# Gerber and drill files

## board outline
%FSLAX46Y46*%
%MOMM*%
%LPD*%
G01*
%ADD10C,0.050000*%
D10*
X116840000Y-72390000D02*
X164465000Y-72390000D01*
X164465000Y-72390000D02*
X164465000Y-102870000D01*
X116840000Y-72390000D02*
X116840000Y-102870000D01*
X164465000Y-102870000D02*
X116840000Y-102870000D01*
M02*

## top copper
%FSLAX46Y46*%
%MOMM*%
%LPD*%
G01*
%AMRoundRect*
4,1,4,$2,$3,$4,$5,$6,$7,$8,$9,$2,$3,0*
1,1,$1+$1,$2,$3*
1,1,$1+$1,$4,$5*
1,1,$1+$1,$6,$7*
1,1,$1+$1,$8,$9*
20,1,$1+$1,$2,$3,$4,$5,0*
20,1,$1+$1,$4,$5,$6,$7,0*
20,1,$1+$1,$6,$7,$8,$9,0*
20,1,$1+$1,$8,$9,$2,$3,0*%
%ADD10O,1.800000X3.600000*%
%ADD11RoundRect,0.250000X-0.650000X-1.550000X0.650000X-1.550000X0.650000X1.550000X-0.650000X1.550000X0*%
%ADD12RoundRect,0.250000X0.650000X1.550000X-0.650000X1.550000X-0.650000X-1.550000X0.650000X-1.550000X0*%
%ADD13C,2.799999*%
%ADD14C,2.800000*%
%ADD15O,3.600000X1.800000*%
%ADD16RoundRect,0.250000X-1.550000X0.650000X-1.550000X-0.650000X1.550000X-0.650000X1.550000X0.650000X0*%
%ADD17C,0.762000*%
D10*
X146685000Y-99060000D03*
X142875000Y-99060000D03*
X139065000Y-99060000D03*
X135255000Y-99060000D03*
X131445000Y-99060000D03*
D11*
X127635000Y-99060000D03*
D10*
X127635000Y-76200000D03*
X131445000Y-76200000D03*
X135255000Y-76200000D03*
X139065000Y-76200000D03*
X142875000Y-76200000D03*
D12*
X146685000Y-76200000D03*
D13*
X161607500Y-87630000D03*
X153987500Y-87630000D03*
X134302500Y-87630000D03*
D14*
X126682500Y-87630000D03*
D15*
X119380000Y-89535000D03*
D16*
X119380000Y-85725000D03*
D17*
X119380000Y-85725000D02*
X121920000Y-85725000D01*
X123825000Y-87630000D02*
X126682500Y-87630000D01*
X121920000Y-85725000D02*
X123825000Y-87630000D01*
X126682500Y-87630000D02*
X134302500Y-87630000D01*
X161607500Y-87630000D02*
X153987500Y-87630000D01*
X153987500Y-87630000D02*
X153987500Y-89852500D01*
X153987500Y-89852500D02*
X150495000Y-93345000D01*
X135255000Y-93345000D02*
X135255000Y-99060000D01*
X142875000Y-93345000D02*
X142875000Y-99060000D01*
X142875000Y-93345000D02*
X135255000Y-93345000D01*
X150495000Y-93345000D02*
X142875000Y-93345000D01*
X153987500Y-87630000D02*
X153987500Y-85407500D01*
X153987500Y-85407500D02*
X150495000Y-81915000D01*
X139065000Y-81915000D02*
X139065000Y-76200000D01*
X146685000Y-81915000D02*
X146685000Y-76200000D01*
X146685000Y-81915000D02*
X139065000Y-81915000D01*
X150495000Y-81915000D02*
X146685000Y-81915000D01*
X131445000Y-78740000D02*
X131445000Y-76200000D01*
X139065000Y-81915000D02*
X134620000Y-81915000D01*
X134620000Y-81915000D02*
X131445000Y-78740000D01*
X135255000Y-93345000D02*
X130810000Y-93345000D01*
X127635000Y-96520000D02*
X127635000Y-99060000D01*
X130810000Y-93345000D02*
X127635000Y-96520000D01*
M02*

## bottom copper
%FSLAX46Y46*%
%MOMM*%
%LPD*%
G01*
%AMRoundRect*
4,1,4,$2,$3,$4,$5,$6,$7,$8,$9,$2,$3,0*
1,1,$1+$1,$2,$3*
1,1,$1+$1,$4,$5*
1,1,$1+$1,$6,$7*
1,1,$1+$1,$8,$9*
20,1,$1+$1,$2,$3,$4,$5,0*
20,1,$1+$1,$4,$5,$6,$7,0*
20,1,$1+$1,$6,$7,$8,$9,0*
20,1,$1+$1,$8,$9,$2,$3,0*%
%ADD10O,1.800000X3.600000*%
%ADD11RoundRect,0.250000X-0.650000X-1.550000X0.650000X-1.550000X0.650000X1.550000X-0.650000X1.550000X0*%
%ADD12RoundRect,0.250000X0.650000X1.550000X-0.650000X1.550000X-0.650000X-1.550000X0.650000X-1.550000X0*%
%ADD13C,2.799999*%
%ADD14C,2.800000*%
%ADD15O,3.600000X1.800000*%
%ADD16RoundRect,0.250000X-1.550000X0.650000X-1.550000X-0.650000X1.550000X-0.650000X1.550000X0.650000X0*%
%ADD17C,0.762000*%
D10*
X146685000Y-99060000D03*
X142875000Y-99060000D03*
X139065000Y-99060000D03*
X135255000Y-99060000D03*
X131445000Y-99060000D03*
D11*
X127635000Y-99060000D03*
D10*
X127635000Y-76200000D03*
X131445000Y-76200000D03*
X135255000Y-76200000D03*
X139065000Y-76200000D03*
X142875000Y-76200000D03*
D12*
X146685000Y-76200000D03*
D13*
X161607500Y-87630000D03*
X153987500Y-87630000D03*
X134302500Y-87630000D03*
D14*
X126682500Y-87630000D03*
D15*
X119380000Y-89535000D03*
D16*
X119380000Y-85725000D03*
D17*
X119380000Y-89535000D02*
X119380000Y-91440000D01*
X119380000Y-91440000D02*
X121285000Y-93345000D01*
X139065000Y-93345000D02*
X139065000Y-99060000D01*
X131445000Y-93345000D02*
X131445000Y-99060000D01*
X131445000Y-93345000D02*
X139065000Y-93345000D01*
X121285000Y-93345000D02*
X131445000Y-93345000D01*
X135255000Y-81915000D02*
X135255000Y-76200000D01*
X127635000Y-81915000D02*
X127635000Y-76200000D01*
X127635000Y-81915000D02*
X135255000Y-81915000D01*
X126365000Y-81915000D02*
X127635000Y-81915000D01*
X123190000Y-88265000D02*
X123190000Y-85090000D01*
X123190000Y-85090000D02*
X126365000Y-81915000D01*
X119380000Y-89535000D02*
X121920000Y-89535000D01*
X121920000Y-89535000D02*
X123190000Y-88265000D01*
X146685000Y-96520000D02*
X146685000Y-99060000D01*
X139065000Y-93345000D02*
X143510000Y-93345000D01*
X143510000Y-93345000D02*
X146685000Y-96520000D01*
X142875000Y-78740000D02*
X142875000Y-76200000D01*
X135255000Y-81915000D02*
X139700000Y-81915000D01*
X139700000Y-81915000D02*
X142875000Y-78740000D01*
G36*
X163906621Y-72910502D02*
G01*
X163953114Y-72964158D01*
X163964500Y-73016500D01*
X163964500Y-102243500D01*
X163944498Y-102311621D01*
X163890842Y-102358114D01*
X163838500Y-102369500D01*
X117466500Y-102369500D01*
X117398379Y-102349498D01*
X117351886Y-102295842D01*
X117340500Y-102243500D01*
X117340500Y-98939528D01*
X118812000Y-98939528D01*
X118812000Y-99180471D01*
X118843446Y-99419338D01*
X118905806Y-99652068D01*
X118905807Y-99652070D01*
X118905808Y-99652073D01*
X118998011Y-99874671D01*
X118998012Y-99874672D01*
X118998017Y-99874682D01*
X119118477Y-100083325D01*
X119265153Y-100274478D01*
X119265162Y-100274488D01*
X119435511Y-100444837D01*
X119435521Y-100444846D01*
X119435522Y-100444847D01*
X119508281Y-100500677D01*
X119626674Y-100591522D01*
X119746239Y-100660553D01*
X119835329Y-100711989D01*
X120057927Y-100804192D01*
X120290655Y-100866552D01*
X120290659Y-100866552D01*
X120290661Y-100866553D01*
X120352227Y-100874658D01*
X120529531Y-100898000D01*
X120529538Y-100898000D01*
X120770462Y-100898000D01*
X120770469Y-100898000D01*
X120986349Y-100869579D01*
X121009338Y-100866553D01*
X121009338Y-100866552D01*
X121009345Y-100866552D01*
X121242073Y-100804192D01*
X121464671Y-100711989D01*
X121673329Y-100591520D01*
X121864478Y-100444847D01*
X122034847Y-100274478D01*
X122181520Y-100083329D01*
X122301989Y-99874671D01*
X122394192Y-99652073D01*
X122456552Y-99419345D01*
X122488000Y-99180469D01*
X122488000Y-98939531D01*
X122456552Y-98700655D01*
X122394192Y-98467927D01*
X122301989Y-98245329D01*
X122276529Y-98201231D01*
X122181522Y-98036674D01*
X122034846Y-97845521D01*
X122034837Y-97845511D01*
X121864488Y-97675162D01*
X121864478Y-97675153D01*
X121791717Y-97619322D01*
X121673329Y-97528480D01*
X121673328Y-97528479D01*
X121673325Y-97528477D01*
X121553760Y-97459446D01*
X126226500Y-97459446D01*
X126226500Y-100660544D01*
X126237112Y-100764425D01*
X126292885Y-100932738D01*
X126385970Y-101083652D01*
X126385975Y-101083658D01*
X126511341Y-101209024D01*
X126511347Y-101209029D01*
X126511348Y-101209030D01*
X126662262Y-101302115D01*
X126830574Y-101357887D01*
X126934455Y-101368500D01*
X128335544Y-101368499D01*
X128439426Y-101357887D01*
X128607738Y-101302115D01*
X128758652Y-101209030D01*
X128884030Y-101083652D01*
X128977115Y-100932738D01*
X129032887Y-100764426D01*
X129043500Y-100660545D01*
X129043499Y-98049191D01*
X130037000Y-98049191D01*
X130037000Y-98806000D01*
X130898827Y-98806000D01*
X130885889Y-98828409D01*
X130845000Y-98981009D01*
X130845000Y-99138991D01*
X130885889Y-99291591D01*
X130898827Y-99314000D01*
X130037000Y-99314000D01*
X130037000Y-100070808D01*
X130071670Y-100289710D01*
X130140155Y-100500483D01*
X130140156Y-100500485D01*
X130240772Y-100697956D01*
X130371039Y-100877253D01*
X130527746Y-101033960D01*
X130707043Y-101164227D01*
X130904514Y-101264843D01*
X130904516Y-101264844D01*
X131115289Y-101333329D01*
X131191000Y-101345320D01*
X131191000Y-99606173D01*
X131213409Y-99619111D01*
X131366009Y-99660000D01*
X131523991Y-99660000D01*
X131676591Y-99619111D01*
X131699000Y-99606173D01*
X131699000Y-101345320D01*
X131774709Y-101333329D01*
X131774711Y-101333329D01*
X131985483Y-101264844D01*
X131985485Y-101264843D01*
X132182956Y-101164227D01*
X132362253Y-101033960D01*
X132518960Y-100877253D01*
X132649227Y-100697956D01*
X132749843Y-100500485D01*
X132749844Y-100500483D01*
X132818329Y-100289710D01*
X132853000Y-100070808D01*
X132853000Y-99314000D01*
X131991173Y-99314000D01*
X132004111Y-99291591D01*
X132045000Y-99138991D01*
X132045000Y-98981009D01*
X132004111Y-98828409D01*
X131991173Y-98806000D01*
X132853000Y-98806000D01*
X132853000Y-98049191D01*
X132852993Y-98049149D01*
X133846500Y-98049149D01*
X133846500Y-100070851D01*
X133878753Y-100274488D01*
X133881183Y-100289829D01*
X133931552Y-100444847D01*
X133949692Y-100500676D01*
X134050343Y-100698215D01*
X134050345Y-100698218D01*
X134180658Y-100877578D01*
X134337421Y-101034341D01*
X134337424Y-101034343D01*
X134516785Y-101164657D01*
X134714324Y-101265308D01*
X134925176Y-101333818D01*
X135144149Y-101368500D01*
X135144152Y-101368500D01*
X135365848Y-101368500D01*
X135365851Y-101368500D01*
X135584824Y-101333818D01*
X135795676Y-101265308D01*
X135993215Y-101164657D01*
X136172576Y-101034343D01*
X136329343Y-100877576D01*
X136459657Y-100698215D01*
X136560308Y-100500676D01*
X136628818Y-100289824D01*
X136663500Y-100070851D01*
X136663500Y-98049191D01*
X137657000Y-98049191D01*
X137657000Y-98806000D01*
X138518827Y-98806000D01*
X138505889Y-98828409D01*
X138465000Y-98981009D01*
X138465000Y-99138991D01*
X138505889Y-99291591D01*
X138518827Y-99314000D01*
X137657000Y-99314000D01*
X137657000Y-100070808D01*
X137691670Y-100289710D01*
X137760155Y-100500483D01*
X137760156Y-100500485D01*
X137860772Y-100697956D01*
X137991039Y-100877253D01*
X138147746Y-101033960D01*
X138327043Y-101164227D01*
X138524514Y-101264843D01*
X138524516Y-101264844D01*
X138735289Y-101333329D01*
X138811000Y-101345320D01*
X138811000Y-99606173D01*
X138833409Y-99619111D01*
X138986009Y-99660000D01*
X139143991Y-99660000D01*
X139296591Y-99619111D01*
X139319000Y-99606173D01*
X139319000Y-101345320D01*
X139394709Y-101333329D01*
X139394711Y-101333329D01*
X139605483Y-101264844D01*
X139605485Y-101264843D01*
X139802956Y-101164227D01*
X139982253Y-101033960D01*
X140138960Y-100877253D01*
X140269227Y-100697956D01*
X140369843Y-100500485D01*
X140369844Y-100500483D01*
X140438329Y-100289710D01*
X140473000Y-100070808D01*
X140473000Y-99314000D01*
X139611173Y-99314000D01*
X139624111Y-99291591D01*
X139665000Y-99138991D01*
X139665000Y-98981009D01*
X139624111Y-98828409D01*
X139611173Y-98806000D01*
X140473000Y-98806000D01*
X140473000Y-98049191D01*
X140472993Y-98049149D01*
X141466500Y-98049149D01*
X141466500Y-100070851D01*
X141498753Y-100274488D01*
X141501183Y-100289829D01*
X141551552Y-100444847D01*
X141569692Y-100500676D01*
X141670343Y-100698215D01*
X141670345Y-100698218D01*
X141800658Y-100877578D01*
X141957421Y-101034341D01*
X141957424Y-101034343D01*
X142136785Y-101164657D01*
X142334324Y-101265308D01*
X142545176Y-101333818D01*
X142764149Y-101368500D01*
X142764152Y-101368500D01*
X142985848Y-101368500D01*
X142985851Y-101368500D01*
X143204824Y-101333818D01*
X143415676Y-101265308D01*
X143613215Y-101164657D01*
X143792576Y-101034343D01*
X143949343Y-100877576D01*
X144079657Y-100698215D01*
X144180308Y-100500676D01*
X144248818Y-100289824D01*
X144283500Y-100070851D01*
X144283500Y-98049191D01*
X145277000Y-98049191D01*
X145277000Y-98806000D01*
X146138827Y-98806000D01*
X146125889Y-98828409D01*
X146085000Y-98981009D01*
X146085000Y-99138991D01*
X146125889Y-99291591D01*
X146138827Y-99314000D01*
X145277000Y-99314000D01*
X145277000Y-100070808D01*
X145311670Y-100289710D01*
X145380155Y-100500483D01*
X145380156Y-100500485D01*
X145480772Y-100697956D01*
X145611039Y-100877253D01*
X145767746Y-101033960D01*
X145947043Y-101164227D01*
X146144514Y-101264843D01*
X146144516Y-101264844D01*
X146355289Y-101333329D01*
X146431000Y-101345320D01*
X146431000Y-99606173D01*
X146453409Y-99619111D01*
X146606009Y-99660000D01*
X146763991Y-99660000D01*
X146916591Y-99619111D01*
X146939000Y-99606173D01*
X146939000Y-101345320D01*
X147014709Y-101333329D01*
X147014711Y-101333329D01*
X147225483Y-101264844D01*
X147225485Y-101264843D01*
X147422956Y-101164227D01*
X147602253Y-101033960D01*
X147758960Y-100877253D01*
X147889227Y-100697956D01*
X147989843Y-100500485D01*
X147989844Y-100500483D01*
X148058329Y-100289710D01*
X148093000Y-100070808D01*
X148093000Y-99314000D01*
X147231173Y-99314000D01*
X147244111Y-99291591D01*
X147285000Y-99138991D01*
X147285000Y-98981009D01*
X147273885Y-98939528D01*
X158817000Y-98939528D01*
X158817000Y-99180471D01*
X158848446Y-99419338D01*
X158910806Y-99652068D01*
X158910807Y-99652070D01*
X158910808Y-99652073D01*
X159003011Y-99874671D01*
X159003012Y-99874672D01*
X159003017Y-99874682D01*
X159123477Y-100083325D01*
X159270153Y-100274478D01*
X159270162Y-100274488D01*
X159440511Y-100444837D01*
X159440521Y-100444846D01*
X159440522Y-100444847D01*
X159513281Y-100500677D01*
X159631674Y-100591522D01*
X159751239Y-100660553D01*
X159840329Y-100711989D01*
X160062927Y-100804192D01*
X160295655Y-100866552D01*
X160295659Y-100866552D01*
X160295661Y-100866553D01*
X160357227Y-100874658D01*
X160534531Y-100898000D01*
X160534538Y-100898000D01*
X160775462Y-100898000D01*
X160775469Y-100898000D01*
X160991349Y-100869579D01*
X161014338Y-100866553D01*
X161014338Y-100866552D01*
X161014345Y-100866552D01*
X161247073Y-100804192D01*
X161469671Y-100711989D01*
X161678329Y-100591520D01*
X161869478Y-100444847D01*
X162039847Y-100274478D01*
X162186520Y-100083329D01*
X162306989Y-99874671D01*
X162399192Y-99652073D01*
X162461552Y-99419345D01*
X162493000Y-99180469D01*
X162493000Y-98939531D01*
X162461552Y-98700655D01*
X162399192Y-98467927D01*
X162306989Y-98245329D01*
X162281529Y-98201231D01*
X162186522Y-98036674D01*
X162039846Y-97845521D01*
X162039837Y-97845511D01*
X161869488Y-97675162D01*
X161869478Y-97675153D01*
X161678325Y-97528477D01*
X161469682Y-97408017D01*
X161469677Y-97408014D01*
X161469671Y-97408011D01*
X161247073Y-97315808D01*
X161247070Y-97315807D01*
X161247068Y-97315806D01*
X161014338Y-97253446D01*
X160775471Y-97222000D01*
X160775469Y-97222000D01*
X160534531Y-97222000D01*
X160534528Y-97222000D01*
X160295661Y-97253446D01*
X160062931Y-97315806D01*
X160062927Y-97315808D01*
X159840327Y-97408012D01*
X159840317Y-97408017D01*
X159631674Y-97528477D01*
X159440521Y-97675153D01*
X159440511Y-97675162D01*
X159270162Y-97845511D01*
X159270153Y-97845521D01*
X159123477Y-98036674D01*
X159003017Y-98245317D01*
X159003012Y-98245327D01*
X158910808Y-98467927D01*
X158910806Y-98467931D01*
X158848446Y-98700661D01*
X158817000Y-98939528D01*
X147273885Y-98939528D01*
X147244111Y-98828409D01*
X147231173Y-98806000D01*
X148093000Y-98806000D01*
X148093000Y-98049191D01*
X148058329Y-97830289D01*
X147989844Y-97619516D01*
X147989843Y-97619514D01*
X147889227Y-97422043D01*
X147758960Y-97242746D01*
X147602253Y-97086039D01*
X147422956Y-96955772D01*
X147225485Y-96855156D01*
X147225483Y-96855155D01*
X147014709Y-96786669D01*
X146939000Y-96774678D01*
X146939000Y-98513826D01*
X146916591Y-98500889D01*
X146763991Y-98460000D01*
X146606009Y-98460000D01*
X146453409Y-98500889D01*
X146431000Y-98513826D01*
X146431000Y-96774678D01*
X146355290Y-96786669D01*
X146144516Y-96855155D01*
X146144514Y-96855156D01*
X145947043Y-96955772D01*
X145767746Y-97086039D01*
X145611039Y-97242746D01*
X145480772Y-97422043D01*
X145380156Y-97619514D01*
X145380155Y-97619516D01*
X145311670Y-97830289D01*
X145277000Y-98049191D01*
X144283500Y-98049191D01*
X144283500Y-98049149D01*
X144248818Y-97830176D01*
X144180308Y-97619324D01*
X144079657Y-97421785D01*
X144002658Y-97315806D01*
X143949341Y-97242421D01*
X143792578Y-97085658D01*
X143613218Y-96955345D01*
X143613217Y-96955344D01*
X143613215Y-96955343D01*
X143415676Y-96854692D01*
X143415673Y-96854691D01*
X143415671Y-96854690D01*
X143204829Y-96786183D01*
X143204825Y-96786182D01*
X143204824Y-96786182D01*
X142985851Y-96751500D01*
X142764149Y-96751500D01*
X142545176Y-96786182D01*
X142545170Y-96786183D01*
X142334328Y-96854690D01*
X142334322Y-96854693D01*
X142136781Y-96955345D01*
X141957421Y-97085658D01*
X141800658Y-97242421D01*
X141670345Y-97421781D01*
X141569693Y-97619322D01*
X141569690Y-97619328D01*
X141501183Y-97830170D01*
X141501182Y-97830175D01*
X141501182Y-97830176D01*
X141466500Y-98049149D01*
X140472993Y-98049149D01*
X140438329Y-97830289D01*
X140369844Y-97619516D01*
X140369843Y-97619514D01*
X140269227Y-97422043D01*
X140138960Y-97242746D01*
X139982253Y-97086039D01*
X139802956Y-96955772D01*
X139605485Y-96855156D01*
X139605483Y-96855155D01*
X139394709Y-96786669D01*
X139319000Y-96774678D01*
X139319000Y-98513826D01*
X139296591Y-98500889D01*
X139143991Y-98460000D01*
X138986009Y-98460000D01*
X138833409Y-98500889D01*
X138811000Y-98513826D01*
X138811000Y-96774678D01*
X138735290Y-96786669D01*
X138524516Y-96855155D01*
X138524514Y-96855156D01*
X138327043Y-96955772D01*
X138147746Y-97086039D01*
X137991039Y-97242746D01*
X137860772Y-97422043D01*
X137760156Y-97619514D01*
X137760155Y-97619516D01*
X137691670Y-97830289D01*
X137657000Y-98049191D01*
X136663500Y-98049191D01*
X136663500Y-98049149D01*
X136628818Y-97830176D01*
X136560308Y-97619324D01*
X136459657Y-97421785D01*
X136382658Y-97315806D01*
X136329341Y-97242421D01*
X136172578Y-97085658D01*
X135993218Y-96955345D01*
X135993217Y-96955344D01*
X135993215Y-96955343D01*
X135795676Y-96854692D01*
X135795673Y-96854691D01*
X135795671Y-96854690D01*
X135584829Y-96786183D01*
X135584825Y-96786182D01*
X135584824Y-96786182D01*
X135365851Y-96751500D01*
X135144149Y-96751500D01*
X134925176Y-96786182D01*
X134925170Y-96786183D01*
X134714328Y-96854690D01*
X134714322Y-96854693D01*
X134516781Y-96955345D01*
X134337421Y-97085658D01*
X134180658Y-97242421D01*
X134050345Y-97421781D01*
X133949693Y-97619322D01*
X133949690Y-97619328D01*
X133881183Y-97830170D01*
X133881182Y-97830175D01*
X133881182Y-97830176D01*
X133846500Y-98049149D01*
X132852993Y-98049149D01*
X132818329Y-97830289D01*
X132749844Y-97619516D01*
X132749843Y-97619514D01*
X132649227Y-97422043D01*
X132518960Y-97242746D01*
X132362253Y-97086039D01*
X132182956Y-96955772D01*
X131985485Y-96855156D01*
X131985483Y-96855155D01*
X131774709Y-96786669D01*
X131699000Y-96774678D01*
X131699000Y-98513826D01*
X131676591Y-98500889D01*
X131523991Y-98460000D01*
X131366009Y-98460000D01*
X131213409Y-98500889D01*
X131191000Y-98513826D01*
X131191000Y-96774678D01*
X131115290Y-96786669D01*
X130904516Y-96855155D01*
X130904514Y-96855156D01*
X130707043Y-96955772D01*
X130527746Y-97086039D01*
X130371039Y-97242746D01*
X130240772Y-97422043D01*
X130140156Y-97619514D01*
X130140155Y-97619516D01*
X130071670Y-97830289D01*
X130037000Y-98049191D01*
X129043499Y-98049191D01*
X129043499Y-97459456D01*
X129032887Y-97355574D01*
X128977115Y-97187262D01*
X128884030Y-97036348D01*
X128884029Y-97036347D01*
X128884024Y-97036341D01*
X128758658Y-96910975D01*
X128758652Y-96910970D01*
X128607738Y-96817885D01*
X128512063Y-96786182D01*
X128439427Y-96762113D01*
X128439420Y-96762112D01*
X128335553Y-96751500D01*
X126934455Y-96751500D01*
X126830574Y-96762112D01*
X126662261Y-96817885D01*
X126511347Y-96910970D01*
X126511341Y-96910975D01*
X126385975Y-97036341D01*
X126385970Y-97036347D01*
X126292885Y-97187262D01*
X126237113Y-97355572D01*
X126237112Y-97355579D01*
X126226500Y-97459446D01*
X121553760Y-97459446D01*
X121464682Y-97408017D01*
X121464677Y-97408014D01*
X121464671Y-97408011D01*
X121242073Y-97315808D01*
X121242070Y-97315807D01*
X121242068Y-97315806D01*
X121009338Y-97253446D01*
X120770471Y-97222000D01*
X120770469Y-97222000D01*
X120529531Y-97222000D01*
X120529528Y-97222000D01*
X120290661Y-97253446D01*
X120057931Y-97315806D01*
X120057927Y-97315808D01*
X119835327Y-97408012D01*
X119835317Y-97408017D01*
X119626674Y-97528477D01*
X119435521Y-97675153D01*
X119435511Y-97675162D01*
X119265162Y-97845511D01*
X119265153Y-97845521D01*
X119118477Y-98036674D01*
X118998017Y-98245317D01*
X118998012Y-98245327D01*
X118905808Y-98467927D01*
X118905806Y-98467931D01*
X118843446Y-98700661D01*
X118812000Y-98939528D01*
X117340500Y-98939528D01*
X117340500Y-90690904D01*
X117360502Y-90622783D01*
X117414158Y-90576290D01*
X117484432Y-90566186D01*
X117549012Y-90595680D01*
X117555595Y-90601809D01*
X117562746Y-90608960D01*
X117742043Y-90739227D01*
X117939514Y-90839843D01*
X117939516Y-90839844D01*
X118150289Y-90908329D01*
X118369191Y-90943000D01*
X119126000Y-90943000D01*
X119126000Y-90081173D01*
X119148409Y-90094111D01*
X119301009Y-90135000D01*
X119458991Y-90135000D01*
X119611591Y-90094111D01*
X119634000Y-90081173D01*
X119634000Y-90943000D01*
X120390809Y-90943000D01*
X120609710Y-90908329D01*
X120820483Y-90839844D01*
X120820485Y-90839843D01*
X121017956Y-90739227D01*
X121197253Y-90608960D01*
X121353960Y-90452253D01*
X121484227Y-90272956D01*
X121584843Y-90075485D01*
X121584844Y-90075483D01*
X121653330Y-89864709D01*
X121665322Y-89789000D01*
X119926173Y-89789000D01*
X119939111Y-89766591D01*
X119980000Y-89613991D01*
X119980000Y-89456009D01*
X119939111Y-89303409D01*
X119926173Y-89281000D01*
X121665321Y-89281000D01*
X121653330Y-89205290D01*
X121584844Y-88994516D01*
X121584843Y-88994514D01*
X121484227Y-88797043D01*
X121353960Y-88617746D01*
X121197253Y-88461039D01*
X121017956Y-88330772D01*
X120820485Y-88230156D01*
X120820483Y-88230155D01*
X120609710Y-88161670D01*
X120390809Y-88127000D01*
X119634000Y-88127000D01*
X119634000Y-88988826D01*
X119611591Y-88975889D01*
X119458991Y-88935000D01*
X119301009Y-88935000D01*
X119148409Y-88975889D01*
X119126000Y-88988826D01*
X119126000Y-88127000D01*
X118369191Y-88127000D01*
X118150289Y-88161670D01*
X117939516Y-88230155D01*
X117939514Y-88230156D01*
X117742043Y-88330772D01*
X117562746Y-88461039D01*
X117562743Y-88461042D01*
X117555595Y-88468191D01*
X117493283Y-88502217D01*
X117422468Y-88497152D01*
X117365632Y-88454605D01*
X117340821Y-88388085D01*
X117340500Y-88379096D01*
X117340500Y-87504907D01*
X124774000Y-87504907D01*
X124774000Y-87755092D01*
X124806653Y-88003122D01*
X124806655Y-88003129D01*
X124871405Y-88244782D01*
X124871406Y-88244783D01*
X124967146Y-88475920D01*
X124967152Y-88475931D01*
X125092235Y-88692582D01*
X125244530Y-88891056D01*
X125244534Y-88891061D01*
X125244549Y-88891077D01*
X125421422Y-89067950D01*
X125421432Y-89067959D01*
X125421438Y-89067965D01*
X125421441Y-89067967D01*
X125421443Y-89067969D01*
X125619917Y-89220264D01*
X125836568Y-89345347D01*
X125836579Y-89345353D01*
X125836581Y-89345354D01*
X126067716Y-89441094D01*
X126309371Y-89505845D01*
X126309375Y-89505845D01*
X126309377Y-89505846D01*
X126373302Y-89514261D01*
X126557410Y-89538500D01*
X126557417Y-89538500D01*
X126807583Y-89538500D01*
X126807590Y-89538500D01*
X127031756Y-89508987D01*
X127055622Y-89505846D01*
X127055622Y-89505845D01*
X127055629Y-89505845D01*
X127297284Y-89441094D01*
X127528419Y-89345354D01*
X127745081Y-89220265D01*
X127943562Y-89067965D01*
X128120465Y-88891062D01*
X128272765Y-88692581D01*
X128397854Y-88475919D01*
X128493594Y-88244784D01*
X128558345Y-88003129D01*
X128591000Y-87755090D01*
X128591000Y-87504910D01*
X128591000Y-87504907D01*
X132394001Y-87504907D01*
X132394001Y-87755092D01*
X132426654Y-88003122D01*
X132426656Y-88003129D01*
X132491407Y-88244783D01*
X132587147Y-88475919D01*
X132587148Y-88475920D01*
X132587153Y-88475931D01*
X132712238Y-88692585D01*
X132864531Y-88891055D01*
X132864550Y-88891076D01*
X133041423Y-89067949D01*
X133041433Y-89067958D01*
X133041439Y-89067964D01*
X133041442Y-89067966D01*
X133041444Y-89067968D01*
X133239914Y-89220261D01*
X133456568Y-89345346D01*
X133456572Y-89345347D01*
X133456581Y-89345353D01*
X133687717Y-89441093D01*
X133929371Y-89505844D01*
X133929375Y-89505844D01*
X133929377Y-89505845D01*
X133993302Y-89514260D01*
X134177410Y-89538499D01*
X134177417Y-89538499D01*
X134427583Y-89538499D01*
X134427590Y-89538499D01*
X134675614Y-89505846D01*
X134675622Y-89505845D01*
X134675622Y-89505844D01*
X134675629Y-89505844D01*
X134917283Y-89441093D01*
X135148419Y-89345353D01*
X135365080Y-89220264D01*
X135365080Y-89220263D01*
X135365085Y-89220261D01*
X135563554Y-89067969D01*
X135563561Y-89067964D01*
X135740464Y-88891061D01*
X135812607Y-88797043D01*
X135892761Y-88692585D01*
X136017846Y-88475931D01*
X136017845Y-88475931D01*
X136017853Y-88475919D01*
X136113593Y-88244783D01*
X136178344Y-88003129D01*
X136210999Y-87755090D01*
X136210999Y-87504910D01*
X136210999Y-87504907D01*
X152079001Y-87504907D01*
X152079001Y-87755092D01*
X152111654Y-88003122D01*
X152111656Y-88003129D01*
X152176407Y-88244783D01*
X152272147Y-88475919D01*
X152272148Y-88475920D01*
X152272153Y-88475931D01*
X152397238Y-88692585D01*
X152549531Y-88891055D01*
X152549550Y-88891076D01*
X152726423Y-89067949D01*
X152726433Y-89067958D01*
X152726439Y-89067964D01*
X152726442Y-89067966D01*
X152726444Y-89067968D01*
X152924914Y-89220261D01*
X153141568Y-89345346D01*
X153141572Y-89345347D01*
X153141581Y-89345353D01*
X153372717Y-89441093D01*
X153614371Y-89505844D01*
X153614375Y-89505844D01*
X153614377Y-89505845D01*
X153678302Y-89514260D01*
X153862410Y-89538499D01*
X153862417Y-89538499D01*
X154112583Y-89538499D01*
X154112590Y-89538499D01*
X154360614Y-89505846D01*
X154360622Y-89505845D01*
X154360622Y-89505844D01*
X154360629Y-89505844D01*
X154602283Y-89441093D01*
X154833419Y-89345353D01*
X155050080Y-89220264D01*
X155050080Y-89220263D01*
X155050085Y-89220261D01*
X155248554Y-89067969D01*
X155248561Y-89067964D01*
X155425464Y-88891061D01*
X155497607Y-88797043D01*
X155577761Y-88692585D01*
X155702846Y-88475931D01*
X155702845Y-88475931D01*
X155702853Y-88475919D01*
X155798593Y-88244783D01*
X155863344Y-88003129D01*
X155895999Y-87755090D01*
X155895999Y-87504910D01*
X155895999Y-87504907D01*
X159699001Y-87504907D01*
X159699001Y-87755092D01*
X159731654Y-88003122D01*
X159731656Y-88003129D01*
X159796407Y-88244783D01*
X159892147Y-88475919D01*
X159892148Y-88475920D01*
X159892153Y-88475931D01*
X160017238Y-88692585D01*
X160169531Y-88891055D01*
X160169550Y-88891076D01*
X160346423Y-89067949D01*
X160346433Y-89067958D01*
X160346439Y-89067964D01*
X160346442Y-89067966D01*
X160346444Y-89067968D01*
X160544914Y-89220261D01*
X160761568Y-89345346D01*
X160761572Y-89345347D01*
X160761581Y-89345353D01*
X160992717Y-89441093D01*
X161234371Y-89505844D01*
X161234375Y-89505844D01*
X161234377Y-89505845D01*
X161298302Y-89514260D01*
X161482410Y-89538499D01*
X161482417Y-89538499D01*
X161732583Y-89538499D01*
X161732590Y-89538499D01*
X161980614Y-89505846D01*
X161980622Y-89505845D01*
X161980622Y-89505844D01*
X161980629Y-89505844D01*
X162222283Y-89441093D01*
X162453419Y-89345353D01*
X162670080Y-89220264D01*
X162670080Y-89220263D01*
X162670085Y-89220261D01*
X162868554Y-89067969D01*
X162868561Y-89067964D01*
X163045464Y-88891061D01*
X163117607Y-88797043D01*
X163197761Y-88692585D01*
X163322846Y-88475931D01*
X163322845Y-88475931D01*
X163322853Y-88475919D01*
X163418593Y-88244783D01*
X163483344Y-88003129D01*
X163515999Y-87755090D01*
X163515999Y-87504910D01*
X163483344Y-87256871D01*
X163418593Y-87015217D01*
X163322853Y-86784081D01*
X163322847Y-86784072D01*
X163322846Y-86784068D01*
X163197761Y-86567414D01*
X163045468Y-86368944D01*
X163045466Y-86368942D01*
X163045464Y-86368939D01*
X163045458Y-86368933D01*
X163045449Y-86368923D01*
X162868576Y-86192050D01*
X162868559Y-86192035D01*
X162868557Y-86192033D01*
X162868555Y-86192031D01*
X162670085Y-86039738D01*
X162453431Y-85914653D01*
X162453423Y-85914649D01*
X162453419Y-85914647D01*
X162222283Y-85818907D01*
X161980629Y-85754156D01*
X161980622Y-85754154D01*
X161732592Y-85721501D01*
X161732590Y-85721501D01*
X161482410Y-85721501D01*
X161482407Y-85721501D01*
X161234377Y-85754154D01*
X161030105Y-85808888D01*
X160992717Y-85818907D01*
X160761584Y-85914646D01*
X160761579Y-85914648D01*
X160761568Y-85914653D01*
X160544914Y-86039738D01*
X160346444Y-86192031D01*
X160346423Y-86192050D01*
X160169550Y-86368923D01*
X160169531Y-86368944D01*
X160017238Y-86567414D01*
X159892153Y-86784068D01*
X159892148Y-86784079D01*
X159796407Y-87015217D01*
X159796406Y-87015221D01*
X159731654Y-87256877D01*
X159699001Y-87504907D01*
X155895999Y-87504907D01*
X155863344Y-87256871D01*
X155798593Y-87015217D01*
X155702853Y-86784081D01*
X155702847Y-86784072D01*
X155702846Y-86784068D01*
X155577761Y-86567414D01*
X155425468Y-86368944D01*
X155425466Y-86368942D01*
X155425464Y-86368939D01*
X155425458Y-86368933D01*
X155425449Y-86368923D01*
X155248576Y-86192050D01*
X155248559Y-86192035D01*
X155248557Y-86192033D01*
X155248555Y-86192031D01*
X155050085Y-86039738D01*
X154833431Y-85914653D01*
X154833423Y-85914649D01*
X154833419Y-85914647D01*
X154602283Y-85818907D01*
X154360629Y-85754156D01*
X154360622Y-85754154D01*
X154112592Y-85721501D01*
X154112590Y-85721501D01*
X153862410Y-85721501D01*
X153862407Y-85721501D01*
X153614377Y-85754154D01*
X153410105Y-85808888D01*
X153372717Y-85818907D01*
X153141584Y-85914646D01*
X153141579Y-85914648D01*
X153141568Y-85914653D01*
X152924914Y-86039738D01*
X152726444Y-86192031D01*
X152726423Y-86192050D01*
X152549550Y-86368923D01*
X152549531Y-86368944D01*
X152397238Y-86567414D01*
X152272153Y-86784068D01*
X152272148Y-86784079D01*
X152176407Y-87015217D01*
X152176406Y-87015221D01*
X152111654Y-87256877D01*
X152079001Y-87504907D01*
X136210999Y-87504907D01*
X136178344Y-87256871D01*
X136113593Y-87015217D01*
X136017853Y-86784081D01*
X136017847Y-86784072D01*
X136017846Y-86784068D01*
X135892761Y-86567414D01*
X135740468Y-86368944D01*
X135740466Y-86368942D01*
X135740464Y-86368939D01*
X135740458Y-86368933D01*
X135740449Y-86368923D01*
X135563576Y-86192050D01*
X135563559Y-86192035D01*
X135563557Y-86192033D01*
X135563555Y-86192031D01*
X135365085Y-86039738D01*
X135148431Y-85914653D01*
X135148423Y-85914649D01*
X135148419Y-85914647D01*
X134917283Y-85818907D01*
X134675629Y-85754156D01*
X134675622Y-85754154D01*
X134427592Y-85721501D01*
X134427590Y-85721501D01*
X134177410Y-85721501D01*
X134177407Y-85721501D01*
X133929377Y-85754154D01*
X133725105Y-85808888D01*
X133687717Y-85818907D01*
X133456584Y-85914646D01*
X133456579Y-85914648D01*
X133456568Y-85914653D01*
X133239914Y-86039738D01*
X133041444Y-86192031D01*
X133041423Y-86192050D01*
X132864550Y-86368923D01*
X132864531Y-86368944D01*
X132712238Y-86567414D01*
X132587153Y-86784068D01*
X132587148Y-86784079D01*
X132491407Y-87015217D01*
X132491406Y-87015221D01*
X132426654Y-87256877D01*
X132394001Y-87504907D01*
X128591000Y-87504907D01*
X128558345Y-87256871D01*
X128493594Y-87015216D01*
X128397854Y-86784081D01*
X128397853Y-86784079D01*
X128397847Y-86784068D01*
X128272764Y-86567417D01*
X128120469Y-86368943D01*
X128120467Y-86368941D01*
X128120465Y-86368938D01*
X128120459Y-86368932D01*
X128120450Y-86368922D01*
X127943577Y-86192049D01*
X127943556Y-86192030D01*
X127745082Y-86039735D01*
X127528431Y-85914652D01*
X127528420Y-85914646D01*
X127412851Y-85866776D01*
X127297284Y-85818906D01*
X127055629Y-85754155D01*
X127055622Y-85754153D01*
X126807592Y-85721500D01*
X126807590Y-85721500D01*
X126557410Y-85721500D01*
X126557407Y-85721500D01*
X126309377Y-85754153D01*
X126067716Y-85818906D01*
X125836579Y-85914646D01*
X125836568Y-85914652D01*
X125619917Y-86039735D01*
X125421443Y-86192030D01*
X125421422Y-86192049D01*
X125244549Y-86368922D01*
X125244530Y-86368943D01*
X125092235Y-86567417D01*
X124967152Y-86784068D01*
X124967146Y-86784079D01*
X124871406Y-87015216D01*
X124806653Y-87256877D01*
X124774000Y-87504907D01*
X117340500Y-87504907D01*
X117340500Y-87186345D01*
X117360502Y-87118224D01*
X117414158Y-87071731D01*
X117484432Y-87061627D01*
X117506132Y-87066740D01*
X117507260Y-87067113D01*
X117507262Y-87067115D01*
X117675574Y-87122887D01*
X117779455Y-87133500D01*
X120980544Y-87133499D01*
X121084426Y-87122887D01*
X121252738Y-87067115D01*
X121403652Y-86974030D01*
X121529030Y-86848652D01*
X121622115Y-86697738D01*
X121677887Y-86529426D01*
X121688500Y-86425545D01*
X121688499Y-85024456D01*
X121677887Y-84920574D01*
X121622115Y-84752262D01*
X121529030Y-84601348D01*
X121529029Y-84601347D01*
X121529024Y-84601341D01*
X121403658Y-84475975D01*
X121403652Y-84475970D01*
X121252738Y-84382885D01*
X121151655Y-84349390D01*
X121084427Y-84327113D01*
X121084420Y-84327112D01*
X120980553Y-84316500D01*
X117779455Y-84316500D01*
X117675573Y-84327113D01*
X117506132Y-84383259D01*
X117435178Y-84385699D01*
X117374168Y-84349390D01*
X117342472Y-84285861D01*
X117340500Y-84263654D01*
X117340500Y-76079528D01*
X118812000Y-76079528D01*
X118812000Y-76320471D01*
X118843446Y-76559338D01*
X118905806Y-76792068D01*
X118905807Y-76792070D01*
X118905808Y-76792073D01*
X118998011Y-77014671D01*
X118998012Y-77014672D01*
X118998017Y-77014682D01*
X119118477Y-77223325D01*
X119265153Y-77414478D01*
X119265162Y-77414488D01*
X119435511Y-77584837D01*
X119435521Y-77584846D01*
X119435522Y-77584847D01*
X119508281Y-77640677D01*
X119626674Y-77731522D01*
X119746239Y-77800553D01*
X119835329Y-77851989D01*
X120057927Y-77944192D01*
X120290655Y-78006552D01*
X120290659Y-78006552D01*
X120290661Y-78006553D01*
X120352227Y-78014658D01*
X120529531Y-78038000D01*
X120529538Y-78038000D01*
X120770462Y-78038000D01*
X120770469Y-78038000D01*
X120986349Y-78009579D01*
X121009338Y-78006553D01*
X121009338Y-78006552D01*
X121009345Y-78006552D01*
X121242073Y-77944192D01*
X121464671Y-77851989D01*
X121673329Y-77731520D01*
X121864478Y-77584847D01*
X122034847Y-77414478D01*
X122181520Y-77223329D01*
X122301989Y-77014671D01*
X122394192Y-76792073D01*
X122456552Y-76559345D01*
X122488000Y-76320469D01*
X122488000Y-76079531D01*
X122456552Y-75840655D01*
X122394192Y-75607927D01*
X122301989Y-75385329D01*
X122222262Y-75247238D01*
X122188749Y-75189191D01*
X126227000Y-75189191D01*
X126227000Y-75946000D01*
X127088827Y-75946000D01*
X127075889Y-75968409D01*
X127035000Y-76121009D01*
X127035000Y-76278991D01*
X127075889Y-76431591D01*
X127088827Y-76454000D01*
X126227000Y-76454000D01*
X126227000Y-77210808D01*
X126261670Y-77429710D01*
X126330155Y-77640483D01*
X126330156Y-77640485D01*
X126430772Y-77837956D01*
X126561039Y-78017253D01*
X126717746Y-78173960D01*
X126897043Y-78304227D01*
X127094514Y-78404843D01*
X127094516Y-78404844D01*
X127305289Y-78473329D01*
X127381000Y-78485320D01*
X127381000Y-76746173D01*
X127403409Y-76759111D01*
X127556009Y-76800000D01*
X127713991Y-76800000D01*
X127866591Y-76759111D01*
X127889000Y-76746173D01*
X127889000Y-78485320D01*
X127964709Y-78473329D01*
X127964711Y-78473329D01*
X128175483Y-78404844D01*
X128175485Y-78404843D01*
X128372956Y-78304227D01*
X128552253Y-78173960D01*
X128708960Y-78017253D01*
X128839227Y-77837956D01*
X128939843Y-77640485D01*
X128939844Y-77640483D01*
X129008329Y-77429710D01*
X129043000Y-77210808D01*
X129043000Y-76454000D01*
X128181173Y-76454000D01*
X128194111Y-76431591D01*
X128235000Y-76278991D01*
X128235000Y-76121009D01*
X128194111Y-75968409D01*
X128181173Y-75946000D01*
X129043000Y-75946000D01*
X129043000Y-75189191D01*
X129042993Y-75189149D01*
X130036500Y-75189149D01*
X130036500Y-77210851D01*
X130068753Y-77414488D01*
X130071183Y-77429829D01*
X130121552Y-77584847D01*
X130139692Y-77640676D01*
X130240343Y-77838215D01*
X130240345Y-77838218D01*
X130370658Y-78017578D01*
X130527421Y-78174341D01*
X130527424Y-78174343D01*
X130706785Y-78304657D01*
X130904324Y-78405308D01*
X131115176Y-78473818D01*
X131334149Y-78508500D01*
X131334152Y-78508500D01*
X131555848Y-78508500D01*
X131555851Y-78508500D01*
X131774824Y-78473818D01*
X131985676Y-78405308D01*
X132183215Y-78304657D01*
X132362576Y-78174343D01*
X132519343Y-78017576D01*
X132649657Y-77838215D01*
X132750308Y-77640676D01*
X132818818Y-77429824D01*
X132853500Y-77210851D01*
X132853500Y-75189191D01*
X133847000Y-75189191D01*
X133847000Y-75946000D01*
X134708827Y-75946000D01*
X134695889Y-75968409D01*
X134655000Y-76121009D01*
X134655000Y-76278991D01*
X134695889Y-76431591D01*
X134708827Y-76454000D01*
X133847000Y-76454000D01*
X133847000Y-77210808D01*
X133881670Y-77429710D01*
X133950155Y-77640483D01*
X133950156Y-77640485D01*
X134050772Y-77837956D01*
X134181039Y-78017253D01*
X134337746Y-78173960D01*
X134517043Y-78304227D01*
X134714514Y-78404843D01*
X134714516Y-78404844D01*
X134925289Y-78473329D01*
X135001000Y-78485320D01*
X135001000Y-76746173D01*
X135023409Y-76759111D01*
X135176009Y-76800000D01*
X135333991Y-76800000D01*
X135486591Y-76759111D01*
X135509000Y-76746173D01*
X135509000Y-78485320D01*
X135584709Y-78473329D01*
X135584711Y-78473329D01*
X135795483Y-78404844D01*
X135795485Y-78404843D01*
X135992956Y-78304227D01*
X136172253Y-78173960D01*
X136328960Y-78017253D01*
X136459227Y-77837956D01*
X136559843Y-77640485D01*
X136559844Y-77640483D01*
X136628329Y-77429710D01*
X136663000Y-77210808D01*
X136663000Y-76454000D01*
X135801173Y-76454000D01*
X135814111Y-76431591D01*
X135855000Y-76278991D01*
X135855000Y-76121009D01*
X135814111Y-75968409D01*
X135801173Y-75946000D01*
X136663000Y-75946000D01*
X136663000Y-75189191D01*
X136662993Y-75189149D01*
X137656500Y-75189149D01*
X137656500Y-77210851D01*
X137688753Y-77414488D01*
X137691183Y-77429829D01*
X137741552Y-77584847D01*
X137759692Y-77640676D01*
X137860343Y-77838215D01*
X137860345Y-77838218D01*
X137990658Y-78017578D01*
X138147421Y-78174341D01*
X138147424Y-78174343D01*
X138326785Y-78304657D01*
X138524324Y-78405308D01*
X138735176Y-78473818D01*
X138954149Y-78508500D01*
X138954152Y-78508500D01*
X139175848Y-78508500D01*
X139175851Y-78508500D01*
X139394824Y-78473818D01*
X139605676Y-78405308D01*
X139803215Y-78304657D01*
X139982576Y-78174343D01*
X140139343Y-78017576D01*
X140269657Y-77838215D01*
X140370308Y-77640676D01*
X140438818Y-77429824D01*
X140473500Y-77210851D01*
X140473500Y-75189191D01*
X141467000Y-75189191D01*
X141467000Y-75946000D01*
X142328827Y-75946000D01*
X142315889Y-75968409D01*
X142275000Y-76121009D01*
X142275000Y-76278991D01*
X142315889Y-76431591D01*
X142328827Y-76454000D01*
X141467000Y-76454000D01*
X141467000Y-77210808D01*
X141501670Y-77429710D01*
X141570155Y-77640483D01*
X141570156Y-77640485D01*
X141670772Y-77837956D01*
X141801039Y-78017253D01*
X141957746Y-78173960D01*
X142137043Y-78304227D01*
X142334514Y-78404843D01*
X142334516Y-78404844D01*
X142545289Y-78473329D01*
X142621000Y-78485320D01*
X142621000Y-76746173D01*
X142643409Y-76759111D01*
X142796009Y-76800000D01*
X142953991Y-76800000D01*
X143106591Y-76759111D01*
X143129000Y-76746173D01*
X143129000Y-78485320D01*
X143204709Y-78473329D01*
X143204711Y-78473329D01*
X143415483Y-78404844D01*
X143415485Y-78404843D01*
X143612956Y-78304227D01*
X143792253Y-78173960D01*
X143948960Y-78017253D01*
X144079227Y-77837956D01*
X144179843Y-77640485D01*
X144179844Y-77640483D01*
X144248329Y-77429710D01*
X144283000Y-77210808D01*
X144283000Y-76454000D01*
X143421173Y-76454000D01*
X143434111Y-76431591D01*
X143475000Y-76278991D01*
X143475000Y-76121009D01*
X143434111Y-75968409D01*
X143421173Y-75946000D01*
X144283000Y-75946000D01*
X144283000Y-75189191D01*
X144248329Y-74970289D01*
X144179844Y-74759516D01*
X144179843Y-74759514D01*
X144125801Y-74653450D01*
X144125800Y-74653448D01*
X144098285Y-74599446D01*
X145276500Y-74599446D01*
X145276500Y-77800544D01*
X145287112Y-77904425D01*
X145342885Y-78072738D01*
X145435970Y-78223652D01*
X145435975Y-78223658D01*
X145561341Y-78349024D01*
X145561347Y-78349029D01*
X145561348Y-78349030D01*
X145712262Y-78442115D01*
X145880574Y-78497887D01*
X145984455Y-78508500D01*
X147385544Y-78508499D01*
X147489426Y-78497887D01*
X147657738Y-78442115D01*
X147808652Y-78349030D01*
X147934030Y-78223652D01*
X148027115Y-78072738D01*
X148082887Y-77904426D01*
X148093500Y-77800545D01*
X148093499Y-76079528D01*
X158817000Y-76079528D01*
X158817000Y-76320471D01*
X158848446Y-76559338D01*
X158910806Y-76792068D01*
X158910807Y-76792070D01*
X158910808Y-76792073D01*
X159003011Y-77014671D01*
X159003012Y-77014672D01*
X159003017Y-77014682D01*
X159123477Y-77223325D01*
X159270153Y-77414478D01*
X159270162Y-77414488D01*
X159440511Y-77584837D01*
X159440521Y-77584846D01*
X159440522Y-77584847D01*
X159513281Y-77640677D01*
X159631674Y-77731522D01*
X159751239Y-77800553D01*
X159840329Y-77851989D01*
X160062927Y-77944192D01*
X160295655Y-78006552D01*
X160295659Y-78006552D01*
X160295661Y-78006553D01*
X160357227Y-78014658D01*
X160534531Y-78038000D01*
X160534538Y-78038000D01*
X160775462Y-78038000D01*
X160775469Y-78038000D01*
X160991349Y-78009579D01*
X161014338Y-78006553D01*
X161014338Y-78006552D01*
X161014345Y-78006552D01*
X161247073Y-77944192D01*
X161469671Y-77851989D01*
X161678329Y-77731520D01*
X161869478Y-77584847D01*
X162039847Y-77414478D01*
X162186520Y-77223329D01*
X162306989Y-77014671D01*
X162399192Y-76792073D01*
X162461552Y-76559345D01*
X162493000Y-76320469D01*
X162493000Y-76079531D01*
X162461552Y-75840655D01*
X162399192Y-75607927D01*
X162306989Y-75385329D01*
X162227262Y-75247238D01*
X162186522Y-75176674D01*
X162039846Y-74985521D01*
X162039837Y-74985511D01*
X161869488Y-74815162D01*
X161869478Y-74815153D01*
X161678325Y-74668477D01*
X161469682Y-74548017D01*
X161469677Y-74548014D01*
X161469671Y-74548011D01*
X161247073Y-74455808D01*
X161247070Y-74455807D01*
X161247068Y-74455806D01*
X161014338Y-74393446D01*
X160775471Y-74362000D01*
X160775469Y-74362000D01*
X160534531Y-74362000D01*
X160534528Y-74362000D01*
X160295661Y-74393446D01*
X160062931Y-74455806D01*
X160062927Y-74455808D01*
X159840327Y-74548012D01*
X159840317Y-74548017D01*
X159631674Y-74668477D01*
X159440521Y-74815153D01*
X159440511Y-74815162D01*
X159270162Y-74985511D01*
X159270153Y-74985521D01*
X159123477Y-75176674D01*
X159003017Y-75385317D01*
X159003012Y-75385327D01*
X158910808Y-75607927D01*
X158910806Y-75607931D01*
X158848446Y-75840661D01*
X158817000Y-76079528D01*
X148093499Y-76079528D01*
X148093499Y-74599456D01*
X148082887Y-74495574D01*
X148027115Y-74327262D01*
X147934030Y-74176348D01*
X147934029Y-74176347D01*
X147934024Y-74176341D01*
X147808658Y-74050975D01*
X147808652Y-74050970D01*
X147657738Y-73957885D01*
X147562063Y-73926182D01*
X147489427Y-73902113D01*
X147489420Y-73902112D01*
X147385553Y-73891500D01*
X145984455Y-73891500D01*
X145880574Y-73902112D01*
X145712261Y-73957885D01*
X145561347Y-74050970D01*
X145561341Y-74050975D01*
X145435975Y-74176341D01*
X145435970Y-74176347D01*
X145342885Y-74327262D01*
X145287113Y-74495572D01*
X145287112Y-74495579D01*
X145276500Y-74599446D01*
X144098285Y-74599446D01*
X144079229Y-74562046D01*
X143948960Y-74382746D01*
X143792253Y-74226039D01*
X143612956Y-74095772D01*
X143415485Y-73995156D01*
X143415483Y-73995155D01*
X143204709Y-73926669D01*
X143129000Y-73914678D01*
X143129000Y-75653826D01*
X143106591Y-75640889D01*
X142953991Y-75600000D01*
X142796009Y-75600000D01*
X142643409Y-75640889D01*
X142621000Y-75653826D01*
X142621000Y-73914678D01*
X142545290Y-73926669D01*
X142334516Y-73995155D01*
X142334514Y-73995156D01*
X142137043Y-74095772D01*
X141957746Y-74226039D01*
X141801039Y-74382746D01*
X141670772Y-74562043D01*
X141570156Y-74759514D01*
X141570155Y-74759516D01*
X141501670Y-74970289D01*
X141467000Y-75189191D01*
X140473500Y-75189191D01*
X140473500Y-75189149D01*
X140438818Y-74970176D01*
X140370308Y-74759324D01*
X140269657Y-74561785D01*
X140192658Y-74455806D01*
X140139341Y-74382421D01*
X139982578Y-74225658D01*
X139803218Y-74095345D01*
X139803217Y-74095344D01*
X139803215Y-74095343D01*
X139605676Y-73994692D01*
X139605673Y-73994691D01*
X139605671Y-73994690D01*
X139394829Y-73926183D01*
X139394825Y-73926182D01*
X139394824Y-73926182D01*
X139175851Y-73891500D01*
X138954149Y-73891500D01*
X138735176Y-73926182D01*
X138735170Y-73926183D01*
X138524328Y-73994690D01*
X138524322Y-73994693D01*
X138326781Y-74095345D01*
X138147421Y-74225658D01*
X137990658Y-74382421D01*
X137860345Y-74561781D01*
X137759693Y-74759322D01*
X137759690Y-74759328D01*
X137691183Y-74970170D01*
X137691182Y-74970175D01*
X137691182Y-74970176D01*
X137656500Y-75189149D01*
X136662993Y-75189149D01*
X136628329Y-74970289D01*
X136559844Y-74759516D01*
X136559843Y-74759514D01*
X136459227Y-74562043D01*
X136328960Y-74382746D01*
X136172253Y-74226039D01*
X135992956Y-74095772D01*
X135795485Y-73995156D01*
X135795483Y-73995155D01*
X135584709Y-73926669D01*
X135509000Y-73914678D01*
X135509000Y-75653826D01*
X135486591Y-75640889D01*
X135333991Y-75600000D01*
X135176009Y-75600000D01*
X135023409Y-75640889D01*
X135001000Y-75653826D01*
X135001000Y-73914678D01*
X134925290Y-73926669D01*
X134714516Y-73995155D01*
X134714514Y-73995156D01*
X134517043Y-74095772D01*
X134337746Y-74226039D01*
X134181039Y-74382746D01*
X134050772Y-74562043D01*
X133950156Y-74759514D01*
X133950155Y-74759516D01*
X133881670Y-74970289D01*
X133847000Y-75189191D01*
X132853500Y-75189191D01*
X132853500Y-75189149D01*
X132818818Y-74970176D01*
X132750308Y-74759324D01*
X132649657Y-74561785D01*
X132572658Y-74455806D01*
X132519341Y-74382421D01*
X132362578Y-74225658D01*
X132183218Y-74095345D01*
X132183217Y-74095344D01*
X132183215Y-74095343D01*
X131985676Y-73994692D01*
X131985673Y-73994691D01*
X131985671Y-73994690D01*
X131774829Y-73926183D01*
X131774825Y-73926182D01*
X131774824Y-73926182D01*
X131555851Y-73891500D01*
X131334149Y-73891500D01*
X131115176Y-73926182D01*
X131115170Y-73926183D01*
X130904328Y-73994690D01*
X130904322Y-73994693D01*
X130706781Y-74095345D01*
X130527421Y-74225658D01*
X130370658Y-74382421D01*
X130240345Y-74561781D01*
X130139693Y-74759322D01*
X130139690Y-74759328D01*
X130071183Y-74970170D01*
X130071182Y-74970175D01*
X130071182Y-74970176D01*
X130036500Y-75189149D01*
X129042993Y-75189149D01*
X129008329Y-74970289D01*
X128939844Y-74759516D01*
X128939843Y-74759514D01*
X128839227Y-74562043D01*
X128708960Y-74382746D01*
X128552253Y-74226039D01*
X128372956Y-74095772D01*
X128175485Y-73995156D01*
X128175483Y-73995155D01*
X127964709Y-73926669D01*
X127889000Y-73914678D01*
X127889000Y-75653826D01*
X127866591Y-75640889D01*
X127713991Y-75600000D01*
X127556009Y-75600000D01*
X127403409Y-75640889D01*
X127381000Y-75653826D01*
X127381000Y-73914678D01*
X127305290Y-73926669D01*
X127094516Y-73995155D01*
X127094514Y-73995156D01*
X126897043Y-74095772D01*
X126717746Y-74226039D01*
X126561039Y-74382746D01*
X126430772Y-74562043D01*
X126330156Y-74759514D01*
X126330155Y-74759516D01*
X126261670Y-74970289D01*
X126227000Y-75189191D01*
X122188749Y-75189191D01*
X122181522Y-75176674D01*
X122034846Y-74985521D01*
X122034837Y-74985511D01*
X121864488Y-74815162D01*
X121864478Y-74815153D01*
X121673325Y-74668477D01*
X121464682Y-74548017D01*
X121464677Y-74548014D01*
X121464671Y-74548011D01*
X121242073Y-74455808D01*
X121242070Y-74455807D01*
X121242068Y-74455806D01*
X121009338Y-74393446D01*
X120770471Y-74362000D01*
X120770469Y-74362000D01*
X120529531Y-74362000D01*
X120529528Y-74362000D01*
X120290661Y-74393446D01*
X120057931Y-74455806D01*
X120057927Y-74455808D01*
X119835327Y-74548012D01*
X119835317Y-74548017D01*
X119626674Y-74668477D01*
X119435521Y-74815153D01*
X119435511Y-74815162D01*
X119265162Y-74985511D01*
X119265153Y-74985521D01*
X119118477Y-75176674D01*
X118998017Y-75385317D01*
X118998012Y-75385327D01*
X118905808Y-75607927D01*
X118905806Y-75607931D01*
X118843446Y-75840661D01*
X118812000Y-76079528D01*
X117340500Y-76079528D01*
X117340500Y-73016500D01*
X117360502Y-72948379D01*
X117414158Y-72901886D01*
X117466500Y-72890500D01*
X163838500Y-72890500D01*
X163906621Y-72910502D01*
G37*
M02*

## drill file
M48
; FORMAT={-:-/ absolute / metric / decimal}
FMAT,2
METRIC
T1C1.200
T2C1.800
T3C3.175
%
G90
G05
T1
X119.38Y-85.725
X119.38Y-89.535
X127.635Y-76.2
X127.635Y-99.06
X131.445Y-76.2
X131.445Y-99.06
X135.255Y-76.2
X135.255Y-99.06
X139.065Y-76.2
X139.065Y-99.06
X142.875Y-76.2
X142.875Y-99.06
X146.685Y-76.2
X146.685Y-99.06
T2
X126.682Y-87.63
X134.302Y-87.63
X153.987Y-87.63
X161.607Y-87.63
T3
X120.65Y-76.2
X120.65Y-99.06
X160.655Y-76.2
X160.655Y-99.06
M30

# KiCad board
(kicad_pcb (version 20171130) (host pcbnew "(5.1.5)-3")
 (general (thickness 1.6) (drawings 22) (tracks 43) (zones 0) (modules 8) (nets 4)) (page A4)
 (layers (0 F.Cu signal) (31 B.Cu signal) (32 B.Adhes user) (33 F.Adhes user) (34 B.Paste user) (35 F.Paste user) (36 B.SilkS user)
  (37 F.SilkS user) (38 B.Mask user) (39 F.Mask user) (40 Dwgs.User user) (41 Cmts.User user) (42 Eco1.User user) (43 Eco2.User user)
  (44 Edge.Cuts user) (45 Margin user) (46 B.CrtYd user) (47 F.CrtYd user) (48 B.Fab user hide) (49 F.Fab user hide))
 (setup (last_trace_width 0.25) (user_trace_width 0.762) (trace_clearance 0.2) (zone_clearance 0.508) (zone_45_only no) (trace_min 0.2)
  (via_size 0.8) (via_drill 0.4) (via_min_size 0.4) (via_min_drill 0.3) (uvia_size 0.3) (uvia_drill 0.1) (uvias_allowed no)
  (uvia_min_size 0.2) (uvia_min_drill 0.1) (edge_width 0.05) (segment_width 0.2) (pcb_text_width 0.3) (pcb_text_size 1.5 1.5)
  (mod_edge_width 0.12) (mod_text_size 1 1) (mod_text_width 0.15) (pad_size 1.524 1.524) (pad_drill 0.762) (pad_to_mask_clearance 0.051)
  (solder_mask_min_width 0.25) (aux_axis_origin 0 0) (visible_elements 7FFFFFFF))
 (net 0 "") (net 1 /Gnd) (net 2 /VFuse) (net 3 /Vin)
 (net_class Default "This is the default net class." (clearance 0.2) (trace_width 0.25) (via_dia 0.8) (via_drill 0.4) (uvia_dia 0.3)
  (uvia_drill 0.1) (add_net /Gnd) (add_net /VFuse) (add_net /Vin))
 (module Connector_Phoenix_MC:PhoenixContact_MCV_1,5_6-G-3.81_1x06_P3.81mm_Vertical (layer F.Cu) (at 127.635 99.06)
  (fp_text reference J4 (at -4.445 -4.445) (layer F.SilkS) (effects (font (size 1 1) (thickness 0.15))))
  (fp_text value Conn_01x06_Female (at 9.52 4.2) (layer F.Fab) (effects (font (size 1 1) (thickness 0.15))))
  (pad 6 thru_hole oval (at 19.05 0) (size 1.8 3.6) (drill 1.2) (layers *.Cu *.Mask) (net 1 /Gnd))
  (pad 5 thru_hole oval (at 15.24 0) (size 1.8 3.6) (drill 1.2) (layers *.Cu *.Mask) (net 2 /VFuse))
  (pad 4 thru_hole oval (at 11.43 0) (size 1.8 3.6) (drill 1.2) (layers *.Cu *.Mask) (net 1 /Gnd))
  (pad 3 thru_hole oval (at 7.62 0) (size 1.8 3.6) (drill 1.2) (layers *.Cu *.Mask) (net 2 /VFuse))
  (pad 2 thru_hole oval (at 3.81 0) (size 1.8 3.6) (drill 1.2) (layers *.Cu *.Mask) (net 1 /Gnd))
  (pad 1 thru_hole roundrect (at 0 0) (size 1.8 3.6) (drill 1.2) (layers *.Cu *.Mask) (roundrect_rratio 0.138889) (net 2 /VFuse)))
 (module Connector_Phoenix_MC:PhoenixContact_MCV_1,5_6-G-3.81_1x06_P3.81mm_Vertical (layer F.Cu) (at 146.685 76.2 180)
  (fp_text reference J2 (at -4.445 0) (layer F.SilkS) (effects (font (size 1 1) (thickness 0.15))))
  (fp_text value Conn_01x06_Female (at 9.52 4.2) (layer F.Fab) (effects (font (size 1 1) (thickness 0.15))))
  (pad 6 thru_hole oval (at 19.05 0 180) (size 1.8 3.6) (drill 1.2) (layers *.Cu *.Mask) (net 1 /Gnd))
  (pad 5 thru_hole oval (at 15.24 0 180) (size 1.8 3.6) (drill 1.2) (layers *.Cu *.Mask) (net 2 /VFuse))
  (pad 4 thru_hole oval (at 11.43 0 180) (size 1.8 3.6) (drill 1.2) (layers *.Cu *.Mask) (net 1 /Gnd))
  (pad 3 thru_hole oval (at 7.62 0 180) (size 1.8 3.6) (drill 1.2) (layers *.Cu *.Mask) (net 2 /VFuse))
  (pad 2 thru_hole oval (at 3.81 0 180) (size 1.8 3.6) (drill 1.2) (layers *.Cu *.Mask) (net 1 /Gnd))
  (pad 1 thru_hole roundrect (at 0 0 180) (size 1.8 3.6) (drill 1.2) (layers *.Cu *.Mask) (roundrect_rratio 0.138889) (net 2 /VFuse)))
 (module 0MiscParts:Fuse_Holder (layer F.Cu) (at 144.145 87.63)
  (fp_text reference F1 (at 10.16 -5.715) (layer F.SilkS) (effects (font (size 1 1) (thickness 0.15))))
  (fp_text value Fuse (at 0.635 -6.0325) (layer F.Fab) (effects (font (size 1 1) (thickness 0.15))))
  (pad 2 thru_hole circle (at 17.4625 0) (size 2.799999 2.799999) (drill 1.8) (layers *.Cu *.Mask) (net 2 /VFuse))
  (pad 2 thru_hole circle (at 9.8425 0) (size 2.799999 2.799999) (drill 1.8) (layers *.Cu *.Mask) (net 2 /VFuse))
  (pad 1 thru_hole circle (at -9.8425 0) (size 2.799999 2.799999) (drill 1.8) (layers *.Cu *.Mask) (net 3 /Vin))
  (pad 1 thru_hole circle (at -17.4625 0) (size 2.8 2.8) (drill 1.8) (layers *.Cu *.Mask) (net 3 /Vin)))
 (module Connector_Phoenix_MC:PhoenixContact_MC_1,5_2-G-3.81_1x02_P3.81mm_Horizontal (layer F.Cu) (at 119.38 85.725 270)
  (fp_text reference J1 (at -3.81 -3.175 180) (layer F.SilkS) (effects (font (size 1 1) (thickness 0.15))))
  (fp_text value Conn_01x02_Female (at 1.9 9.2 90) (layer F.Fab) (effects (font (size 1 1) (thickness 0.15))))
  (pad 2 thru_hole oval (at 3.81 0 270) (size 1.8 3.6) (drill 1.2) (layers *.Cu *.Mask) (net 1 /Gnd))
  (pad 1 thru_hole roundrect (at 0 0 270) (size 1.8 3.6) (drill 1.2) (layers *.Cu *.Mask) (roundrect_rratio 0.138889) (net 3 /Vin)))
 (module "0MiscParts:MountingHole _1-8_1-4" (layer F.Cu) (at 160.655 99.06)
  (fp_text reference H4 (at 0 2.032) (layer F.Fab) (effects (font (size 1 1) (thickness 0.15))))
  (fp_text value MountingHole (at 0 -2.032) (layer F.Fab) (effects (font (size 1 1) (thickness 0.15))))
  (pad "" np_thru_hole circle (at 0 0) (size 3.175 3.175) (drill 3.175) (layers *.Cu *.Mask)))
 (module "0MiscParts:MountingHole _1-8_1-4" (layer F.Cu) (at 160.655 76.2)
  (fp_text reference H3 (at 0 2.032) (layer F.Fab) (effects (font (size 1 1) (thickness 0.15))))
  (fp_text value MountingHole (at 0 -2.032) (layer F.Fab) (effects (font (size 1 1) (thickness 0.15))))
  (pad "" np_thru_hole circle (at 0 0) (size 3.175 3.175) (drill 3.175) (layers *.Cu *.Mask)))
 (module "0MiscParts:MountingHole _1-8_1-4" (layer F.Cu) (at 120.65 76.2)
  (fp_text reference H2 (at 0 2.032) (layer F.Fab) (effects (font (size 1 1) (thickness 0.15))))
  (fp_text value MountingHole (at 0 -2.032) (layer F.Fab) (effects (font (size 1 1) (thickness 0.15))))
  (pad "" np_thru_hole circle (at 0 0) (size 3.175 3.175) (drill 3.175) (layers *.Cu *.Mask)))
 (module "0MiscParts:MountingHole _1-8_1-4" (layer F.Cu) (at 120.65 99.06 90)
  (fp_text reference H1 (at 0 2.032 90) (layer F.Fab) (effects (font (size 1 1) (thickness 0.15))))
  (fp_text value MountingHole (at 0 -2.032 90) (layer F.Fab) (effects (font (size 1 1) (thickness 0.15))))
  (pad "" np_thru_hole circle (at 0 0 90) (size 3.175 3.175) (drill 3.175) (layers *.Cu *.Mask)))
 (gr_line (start 116.84 72.39) (end 164.465 72.39) (layer Edge.Cuts) (width 0.05))
 (gr_line (start 164.465 72.39) (end 164.465 102.87) (layer Edge.Cuts) (width 0.05))
 (gr_line (start 116.84 72.39) (end 116.84 102.87) (layer Edge.Cuts) (width 0.05))
 (gr_line (start 164.465 102.87) (end 116.84 102.87) (layer Edge.Cuts) (width 0.05))
 (segment (start 119.38 85.725) (end 121.92 85.725) (width 0.762) (layer F.Cu) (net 3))
 (segment (start 123.825 87.63) (end 126.6825 87.63) (width 0.762) (layer F.Cu) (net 3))
 (segment (start 121.92 85.725) (end 123.825 87.63) (width 0.762) (layer F.Cu) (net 3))
 (segment (start 126.6825 87.63) (end 134.3025 87.63) (width 0.762) (layer F.Cu) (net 3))
 (segment (start 119.38 89.535) (end 119.38 91.44) (width 0.762) (layer B.Cu) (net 1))
 (segment (start 119.38 91.44) (end 121.285 93.345) (width 0.762) (layer B.Cu) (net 1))
 (segment (start 139.065 93.345) (end 139.065 99.06) (width 0.762) (layer B.Cu) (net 1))
 (segment (start 131.445 93.345) (end 131.445 99.06) (width 0.762) (layer B.Cu) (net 1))
 (segment (start 131.445 93.345) (end 139.065 93.345) (width 0.762) (layer B.Cu) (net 1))
 (segment (start 121.285 93.345) (end 131.445 93.345) (width 0.762) (layer B.Cu) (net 1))
 (segment (start 135.255 81.915) (end 135.255 76.2) (width 0.762) (layer B.Cu) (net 1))
 (segment (start 127.635 81.915) (end 127.635 76.2) (width 0.762) (layer B.Cu) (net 1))
 (segment (start 127.635 81.915) (end 135.255 81.915) (width 0.762) (layer B.Cu) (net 1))
 (segment (start 126.365 81.915) (end 127.635 81.915) (width 0.762) (layer B.Cu) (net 1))
 (segment (start 123.19 88.265) (end 123.19 85.09) (width 0.762) (layer B.Cu) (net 1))
 (segment (start 123.19 85.09) (end 126.365 81.915) (width 0.762) (layer B.Cu) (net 1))
 (segment (start 119.38 89.535) (end 121.92 89.535) (width 0.762) (layer B.Cu) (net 1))
 (segment (start 121.92 89.535) (end 123.19 88.265) (width 0.762) (layer B.Cu) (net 1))
 (segment (start 146.685 96.52) (end 146.685 99.06) (width 0.762) (layer B.Cu) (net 1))
 (segment (start 139.065 93.345) (end 143.51 93.345) (width 0.762) (layer B.Cu) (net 1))
 (segment (start 143.51 93.345) (end 146.685 96.52) (width 0.762) (layer B.Cu) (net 1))
 (segment (start 142.875 78.74) (end 142.875 76.2) (width 0.762) (layer B.Cu) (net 1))
 (segment (start 135.255 81.915) (end 139.7 81.915) (width 0.762) (layer B.Cu) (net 1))
 (segment (start 139.7 81.915) (end 142.875 78.74) (width 0.762) (layer B.Cu) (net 1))
 (segment (start 161.6075 87.63) (end 153.9875 87.63) (width 0.762) (layer F.Cu) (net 2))
 (segment (start 153.9875 87.63) (end 153.9875 89.8525) (width 0.762) (layer F.Cu) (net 2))
 (segment (start 153.9875 89.8525) (end 150.495 93.345) (width 0.762) (layer F.Cu) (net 2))
 (segment (start 135.255 93.345) (end 135.255 99.06) (width 0.762) (layer F.Cu) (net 2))
 (segment (start 142.875 93.345) (end 142.875 99.06) (width 0.762) (layer F.Cu) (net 2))
 (segment (start 142.875 93.345) (end 135.255 93.345) (width 0.762) (layer F.Cu) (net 2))
 (segment (start 150.495 93.345) (end 142.875 93.345) (width 0.762) (layer F.Cu) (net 2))
 (segment (start 153.9875 87.63) (end 153.9875 85.4075) (width 0.762) (layer F.Cu) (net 2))
 (segment (start 153.9875 85.4075) (end 150.495 81.915) (width 0.762) (layer F.Cu) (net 2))
 (segment (start 139.065 81.915) (end 139.065 76.2) (width 0.762) (layer F.Cu) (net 2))
 (segment (start 146.685 81.915) (end 146.685 76.2) (width 0.762) (layer F.Cu) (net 2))
 (segment (start 146.685 81.915) (end 139.065 81.915) (width 0.762) (layer F.Cu) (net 2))
 (segment (start 150.495 81.915) (end 146.685 81.915) (width 0.762) (layer F.Cu) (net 2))
 (segment (start 131.445 78.74) (end 131.445 76.2) (width 0.762) (layer F.Cu) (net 2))
 (segment (start 139.065 81.915) (end 134.62 81.915) (width 0.762) (layer F.Cu) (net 2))
 (segment (start 134.62 81.915) (end 131.445 78.74) (width 0.762) (layer F.Cu) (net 2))
 (segment (start 135.255 93.345) (end 130.81 93.345) (width 0.762) (layer F.Cu) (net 2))
 (segment (start 127.635 96.52) (end 127.635 99.06) (width 0.762) (layer F.Cu) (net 2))
 (segment (start 130.81 93.345) (end 127.635 96.52) (width 0.762) (layer F.Cu) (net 2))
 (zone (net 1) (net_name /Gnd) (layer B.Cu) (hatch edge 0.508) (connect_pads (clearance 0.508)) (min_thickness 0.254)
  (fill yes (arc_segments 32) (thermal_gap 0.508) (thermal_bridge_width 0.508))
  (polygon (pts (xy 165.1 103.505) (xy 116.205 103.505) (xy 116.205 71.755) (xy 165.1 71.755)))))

